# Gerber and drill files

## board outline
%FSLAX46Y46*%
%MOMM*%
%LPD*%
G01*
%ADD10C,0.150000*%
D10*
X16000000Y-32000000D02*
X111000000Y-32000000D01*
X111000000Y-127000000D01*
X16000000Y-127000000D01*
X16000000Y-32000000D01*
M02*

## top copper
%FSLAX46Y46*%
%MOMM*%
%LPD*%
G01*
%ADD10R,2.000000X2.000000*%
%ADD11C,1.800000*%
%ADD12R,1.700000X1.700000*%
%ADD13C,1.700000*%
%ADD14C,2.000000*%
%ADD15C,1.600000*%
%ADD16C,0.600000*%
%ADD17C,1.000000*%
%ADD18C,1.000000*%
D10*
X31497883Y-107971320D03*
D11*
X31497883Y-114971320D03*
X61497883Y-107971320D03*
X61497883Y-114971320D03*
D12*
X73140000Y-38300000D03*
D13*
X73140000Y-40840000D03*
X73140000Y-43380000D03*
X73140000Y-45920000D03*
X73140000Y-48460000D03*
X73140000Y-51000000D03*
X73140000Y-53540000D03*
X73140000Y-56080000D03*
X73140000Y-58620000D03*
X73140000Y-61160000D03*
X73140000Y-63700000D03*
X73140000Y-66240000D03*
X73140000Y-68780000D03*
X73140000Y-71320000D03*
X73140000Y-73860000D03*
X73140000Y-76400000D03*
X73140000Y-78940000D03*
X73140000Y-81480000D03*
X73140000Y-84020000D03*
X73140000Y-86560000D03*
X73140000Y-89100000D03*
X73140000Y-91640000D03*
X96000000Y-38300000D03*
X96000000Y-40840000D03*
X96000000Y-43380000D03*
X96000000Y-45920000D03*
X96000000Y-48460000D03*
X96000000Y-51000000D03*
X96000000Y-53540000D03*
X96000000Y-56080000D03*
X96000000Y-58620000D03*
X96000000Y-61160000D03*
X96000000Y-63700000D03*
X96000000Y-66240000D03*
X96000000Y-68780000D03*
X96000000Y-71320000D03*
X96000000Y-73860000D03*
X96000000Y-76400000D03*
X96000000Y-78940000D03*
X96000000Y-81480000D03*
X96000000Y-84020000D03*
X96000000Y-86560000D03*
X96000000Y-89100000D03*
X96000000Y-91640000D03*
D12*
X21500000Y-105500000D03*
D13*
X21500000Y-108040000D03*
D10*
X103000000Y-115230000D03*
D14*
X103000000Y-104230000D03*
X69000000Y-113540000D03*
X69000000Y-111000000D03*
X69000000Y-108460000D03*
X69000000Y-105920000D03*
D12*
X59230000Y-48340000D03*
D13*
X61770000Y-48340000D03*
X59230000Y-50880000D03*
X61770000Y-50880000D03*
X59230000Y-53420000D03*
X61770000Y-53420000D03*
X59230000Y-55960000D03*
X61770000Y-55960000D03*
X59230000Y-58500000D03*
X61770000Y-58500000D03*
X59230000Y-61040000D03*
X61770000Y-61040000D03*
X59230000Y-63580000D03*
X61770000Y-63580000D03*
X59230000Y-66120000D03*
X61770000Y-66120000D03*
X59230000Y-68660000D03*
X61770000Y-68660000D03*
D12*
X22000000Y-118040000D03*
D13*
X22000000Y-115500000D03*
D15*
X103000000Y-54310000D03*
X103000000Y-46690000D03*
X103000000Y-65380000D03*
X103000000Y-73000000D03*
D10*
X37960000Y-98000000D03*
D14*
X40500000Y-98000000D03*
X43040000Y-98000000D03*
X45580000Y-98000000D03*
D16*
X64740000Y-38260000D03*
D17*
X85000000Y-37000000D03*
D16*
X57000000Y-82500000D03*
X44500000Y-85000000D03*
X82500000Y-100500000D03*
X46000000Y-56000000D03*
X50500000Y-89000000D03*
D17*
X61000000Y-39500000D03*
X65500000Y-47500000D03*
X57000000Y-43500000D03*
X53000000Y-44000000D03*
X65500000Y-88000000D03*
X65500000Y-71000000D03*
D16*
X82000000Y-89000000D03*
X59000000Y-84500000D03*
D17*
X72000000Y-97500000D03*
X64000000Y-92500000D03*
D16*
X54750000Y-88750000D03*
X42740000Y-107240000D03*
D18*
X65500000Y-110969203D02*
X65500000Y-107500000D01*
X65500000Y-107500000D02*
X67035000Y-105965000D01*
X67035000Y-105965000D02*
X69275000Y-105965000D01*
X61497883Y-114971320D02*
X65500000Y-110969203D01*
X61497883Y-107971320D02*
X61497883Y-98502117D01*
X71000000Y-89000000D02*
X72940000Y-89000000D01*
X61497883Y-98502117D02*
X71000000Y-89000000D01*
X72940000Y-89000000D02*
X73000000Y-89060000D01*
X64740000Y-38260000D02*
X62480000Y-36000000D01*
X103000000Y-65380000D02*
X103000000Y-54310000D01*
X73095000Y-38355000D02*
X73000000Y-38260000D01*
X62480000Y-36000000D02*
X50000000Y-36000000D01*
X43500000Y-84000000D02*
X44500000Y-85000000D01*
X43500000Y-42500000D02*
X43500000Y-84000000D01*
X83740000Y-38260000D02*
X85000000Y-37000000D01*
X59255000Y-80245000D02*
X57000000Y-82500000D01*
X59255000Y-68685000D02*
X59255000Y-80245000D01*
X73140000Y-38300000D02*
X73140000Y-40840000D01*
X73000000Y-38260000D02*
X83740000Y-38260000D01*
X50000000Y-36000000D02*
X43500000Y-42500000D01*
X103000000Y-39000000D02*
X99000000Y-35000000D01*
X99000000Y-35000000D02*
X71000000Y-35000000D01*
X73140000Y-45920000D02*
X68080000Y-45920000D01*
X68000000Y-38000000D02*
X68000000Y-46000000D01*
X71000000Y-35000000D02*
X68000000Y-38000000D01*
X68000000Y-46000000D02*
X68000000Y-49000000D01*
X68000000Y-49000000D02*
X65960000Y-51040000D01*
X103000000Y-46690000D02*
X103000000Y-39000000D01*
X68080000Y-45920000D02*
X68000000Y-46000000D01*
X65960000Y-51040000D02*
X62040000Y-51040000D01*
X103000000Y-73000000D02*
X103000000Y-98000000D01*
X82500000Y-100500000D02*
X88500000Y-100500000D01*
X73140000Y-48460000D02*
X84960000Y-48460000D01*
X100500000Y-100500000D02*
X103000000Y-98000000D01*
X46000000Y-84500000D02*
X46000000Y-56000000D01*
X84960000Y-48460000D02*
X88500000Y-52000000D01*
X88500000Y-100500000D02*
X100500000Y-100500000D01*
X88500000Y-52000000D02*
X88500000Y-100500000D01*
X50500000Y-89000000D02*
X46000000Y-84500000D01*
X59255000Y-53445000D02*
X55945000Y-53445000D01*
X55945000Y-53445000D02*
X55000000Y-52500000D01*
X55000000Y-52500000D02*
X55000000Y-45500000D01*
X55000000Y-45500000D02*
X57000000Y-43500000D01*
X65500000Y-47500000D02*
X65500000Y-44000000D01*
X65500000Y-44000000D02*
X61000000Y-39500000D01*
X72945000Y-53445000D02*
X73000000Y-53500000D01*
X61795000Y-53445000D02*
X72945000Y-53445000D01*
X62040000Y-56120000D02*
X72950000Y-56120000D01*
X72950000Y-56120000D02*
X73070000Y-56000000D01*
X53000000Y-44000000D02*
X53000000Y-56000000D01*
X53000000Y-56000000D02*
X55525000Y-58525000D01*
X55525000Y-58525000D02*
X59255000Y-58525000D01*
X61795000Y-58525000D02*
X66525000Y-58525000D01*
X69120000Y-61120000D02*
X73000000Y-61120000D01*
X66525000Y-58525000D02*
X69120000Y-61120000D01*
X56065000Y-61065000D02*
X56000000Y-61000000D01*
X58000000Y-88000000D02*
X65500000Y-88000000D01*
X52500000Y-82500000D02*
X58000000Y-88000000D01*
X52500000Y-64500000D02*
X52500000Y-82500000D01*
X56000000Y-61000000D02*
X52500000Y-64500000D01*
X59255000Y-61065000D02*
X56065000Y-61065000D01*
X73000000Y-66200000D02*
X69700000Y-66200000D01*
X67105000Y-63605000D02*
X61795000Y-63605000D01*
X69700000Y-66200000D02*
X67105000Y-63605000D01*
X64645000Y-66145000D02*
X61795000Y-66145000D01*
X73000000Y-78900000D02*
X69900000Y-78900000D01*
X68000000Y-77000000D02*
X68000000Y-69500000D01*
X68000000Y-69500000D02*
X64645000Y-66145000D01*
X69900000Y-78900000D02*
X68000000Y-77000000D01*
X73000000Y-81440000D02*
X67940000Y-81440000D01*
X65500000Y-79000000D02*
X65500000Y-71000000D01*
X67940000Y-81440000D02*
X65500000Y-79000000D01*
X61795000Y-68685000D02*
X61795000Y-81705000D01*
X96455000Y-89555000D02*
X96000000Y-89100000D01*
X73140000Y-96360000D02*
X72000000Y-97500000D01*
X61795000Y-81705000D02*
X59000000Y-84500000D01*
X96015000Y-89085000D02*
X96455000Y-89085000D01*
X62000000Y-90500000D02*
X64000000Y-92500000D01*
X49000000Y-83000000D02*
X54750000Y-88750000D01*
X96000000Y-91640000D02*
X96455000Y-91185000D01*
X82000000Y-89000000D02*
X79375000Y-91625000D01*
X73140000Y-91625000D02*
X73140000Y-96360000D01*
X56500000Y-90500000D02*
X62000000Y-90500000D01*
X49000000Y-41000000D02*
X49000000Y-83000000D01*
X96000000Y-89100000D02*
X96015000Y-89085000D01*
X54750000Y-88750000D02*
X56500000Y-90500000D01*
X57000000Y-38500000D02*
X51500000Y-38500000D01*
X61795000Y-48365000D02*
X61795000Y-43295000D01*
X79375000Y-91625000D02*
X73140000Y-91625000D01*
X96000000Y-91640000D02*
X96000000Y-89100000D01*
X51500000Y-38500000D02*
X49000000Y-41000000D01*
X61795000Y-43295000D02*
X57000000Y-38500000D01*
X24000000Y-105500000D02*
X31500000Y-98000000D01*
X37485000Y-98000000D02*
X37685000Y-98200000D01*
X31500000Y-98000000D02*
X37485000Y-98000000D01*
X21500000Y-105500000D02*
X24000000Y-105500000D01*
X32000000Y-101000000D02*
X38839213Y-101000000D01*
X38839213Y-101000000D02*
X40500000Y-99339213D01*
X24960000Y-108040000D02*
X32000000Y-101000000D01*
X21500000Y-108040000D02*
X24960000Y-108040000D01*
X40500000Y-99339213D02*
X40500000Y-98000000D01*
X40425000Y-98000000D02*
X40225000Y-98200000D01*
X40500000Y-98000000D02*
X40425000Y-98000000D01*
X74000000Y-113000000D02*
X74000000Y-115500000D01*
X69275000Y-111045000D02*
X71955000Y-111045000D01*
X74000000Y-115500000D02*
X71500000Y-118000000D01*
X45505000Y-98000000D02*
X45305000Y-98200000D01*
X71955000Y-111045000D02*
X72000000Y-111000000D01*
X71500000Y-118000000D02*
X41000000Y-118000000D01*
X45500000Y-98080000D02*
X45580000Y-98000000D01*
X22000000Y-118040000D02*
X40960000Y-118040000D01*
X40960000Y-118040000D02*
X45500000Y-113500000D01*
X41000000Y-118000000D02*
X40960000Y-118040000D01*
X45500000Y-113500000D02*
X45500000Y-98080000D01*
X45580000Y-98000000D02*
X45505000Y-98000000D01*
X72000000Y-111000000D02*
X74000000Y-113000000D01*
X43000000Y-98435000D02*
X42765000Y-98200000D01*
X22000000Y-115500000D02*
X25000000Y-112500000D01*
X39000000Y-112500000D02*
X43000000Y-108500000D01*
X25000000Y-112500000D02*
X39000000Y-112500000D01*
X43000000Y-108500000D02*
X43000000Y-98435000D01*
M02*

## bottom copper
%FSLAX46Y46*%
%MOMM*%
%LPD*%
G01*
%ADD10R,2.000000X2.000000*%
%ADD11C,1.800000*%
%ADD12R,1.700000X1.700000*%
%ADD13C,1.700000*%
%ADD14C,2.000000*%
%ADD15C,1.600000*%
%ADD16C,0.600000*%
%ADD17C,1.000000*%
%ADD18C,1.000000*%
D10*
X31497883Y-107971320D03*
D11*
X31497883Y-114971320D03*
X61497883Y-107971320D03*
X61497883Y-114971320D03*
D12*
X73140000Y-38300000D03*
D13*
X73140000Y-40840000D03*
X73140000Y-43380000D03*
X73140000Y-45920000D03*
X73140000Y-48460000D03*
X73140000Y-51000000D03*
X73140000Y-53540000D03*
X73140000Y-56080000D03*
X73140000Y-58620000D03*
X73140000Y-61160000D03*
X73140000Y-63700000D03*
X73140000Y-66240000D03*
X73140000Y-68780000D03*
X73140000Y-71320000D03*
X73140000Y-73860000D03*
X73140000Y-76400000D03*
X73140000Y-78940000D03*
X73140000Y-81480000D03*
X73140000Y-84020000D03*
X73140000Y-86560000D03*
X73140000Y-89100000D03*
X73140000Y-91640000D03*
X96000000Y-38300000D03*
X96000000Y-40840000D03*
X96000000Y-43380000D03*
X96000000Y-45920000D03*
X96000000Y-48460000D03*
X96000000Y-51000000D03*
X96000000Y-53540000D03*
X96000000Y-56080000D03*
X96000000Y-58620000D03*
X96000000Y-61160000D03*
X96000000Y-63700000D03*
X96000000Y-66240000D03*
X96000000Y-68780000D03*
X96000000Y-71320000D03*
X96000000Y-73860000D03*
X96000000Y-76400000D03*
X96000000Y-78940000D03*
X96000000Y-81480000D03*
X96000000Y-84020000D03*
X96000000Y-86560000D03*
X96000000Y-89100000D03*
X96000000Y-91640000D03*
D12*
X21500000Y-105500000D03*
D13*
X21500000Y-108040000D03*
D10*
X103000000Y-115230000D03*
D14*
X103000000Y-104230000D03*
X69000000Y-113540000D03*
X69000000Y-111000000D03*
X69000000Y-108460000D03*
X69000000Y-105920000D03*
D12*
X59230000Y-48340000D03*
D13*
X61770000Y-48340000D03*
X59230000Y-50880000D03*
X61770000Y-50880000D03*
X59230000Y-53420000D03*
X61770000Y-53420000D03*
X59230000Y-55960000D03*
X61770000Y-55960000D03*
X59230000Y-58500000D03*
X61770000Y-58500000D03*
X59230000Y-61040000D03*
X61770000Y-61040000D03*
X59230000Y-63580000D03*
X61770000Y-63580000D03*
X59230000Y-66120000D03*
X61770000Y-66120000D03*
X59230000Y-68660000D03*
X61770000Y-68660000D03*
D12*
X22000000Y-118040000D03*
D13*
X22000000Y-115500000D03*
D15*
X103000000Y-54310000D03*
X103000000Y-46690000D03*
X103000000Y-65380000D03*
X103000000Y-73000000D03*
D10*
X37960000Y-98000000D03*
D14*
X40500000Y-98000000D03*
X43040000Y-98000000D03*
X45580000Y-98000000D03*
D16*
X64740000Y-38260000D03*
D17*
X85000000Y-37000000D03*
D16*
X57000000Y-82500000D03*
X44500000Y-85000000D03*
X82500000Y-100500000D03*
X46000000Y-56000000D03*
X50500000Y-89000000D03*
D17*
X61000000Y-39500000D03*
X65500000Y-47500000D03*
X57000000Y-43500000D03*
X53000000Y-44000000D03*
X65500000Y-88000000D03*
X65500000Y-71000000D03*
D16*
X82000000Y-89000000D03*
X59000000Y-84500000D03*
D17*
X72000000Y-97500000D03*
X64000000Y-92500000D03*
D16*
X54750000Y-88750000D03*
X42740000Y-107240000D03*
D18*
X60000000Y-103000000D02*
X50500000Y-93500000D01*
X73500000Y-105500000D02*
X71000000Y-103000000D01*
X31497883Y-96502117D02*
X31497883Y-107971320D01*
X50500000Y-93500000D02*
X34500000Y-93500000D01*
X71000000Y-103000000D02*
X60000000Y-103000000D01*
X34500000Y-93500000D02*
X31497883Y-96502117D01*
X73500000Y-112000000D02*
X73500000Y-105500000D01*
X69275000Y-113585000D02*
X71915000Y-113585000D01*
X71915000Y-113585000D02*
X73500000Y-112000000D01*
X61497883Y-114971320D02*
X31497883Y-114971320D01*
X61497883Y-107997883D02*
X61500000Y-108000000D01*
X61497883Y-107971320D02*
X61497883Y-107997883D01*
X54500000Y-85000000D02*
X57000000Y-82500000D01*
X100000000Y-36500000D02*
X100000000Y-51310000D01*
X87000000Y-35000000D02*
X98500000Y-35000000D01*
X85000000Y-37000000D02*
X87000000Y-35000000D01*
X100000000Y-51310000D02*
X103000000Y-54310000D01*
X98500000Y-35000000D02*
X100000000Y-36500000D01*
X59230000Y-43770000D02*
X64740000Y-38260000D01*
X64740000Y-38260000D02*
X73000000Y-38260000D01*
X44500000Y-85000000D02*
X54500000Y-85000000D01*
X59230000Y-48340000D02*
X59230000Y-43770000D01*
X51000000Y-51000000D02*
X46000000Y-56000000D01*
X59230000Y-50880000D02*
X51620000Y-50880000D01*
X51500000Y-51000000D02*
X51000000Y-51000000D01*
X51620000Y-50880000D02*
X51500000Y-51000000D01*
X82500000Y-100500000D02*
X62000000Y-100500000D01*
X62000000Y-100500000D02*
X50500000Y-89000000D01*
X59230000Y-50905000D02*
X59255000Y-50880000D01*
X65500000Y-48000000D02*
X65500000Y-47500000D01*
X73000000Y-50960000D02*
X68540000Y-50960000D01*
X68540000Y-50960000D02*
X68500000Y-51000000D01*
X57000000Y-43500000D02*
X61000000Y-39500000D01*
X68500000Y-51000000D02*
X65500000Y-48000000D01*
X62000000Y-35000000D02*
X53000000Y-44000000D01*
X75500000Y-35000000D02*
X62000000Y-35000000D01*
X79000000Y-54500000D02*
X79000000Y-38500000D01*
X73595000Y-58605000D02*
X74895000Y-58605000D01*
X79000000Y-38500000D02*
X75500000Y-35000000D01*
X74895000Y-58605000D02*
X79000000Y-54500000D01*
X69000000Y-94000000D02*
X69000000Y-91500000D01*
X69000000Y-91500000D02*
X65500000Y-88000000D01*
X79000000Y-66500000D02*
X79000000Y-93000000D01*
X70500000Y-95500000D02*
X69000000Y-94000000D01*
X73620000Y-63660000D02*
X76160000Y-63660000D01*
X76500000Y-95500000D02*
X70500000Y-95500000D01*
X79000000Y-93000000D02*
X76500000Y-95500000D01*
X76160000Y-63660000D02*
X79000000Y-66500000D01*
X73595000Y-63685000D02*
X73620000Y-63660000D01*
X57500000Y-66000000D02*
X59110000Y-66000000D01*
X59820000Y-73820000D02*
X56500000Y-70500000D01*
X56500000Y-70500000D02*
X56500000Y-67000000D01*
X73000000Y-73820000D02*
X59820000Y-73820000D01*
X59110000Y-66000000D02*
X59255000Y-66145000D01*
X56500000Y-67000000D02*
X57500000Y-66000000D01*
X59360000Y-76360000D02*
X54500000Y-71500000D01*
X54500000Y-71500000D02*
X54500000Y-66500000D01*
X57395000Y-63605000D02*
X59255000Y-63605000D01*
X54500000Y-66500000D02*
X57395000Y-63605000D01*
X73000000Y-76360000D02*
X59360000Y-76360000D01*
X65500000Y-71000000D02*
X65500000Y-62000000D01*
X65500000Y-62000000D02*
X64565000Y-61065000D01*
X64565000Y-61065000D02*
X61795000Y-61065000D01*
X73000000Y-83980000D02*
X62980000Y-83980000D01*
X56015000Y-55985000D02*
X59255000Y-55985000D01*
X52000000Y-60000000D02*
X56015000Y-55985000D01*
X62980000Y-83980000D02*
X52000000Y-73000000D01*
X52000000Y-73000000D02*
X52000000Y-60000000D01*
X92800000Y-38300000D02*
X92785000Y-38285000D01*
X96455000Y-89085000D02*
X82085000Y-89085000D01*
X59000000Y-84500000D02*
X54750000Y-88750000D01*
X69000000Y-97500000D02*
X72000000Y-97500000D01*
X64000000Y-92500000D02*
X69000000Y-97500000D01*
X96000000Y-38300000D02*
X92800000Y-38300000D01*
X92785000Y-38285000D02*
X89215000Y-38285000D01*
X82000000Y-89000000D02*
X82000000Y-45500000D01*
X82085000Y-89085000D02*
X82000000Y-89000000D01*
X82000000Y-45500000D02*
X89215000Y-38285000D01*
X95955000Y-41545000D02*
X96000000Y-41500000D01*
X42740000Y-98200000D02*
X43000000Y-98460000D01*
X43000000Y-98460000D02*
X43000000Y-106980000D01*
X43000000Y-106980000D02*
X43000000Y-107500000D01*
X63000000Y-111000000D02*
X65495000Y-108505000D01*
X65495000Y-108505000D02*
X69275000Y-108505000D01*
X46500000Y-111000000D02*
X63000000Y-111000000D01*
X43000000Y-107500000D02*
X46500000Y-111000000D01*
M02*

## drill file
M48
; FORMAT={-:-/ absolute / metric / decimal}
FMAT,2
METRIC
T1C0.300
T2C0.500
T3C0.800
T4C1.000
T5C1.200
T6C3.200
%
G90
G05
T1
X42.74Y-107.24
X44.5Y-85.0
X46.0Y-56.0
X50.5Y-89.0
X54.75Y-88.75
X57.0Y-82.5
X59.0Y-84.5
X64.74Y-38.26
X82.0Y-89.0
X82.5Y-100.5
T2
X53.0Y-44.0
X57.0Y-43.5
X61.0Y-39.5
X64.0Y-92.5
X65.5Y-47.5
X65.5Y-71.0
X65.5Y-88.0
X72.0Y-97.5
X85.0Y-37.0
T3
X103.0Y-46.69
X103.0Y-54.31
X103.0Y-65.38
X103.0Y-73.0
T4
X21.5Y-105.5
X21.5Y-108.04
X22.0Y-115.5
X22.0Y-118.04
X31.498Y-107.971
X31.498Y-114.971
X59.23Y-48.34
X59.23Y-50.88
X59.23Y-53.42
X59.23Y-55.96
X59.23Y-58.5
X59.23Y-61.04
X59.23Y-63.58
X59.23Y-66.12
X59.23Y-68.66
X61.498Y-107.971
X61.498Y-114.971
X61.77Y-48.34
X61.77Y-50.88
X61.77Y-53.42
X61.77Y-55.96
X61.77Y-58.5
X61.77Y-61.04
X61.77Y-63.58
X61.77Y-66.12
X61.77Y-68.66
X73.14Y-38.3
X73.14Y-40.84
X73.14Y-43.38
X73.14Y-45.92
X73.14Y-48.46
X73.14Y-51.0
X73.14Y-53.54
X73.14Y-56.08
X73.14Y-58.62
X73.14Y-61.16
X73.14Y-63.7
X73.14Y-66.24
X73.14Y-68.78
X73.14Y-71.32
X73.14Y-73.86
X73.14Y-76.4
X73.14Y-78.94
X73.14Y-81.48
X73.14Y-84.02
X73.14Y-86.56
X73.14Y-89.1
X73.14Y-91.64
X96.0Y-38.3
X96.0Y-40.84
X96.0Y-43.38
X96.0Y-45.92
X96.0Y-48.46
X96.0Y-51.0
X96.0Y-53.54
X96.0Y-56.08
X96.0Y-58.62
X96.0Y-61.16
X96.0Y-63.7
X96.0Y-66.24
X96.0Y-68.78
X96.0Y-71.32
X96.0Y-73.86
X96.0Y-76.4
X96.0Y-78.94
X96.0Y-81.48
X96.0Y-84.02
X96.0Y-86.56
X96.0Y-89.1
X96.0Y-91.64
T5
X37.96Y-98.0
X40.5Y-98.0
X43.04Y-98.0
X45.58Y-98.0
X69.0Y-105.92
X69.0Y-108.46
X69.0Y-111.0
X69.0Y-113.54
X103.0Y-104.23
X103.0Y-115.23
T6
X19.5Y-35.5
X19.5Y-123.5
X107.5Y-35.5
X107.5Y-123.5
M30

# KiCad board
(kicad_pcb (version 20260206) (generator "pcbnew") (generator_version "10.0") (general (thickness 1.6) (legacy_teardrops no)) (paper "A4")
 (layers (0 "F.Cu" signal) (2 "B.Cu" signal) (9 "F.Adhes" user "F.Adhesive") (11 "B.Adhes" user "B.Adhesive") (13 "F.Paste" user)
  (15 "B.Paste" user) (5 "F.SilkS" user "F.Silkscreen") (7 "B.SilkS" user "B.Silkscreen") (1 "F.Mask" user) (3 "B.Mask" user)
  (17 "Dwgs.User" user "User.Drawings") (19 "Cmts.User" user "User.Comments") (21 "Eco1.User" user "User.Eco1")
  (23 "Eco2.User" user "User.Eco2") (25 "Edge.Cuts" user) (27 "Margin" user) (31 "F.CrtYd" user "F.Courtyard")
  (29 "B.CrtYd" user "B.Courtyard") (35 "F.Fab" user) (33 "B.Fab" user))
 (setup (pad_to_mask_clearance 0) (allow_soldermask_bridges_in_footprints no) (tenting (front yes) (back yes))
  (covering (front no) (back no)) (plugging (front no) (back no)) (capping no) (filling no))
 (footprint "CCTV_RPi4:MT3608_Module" (layer "F.Cu") (at 46.497883 111.47132)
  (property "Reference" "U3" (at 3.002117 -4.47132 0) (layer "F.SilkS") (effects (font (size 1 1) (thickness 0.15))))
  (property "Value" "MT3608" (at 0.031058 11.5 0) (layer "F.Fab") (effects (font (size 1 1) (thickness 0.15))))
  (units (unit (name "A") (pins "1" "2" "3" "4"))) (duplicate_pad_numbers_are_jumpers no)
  (pad "1" thru_hole rect (at -15 -3.5) (size 2 2) (drill 1) (layers "*.Cu" "*.Mask") (remove_unused_layers no) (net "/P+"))
  (pad "2" thru_hole circle (at -15 3.5) (size 1.8 1.8) (drill 1) (layers "*.Cu" "*.Mask") (remove_unused_layers no) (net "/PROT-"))
  (pad "3" thru_hole circle (at 15 -3.5) (size 1.8 1.8) (drill 1) (layers "*.Cu" "*.Mask") (remove_unused_layers no) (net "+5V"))
  (pad "4" thru_hole circle (at 15 3.5) (size 1.8 1.8) (drill 1) (layers "*.Cu" "*.Mask") (remove_unused_layers no) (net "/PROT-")))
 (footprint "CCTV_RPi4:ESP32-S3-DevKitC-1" (layer "F.Cu") (at 84.57 66.24)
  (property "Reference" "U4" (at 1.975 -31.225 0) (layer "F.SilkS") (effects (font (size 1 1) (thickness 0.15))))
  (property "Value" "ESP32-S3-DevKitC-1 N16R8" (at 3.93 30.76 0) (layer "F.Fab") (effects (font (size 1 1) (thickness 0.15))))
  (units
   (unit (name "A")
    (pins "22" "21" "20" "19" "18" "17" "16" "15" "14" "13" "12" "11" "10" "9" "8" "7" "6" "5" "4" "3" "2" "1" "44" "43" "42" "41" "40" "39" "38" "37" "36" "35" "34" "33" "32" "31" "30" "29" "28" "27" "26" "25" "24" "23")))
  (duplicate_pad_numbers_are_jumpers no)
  (pad "1" thru_hole rect (at -11.43 -27.94) (size 1.7 1.7) (drill 1) (layers "*.Cu" "*.Mask") (remove_unused_layers no) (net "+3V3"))
  (pad "2" thru_hole circle (at -11.43 -25.4) (size 1.7 1.7) (drill 1) (layers "*.Cu" "*.Mask") (remove_unused_layers no) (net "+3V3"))
  (pad "3" thru_hole circle (at -11.43 -22.86) (size 1.7 1.7) (drill 1) (layers "*.Cu" "*.Mask") (remove_unused_layers no)
   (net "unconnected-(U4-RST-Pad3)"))
  (pad "4" thru_hole circle (at -11.43 -20.32) (size 1.7 1.7) (drill 1) (layers "*.Cu" "*.Mask") (remove_unused_layers no) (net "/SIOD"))
  (pad "5" thru_hole circle (at -11.43 -17.78) (size 1.7 1.7) (drill 1) (layers "*.Cu" "*.Mask") (remove_unused_layers no) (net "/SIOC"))
  (pad "6" thru_hole circle (at -11.43 -15.24) (size 1.7 1.7) (drill 1) (layers "*.Cu" "*.Mask") (remove_unused_layers no) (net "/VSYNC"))
  (pad "7" thru_hole circle (at -11.43 -12.7) (size 1.7 1.7) (drill 1) (layers "*.Cu" "*.Mask") (remove_unused_layers no) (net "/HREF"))
  (pad "8" thru_hole circle (at -11.43 -10.16) (size 1.7 1.7) (drill 1) (layers "*.Cu" "*.Mask") (remove_unused_layers no) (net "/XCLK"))
  (pad "9" thru_hole circle (at -11.43 -7.62) (size 1.7 1.7) (drill 1) (layers "*.Cu" "*.Mask") (remove_unused_layers no) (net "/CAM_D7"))
  (pad "10" thru_hole circle (at -11.43 -5.08) (size 1.7 1.7) (drill 1) (layers "*.Cu" "*.Mask") (remove_unused_layers no) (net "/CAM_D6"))
  (pad "11" thru_hole circle (at -11.43 -2.54) (size 1.7 1.7) (drill 1) (layers "*.Cu" "*.Mask") (remove_unused_layers no) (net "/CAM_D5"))
  (pad "12" thru_hole circle (at -11.43 0) (size 1.7 1.7) (drill 1) (layers "*.Cu" "*.Mask") (remove_unused_layers no) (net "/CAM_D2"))
  (pad "13" thru_hole circle (at -11.43 2.54) (size 1.7 1.7) (drill 1) (layers "*.Cu" "*.Mask") (remove_unused_layers no)
   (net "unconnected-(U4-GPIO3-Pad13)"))
  (pad "14" thru_hole circle (at -11.43 5.08) (size 1.7 1.7) (drill 1) (layers "*.Cu" "*.Mask") (remove_unused_layers no)
   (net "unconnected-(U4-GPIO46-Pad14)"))
  (pad "15" thru_hole circle (at -11.43 7.62) (size 1.7 1.7) (drill 1) (layers "*.Cu" "*.Mask") (remove_unused_layers no) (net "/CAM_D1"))
  (pad "16" thru_hole circle (at -11.43 10.16) (size 1.7 1.7) (drill 1) (layers "*.Cu" "*.Mask") (remove_unused_layers no) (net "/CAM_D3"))
  (pad "17" thru_hole circle (at -11.43 12.7) (size 1.7 1.7) (drill 1) (layers "*.Cu" "*.Mask") (remove_unused_layers no) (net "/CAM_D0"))
  (pad "18" thru_hole circle (at -11.43 15.24) (size 1.7 1.7) (drill 1) (layers "*.Cu" "*.Mask") (remove_unused_layers no) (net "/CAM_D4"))
  (pad "19" thru_hole circle (at -11.43 17.78) (size 1.7 1.7) (drill 1) (layers "*.Cu" "*.Mask") (remove_unused_layers no) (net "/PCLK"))
  (pad "20" thru_hole circle (at -11.43 20.32) (size 1.7 1.7) (drill 1) (layers "*.Cu" "*.Mask") (remove_unused_layers no)
   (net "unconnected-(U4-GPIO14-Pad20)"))
  (pad "21" thru_hole circle (at -11.43 22.86) (size 1.7 1.7) (drill 1) (layers "*.Cu" "*.Mask") (remove_unused_layers no) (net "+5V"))
  (pad "22" thru_hole circle (at -11.43 25.4) (size 1.7 1.7) (drill 1) (layers "*.Cu" "*.Mask") (remove_unused_layers no) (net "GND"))
  (pad "23" thru_hole circle (at 11.43 -27.94) (size 1.7 1.7) (drill 1) (layers "*.Cu" "*.Mask") (remove_unused_layers no) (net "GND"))
  (pad "24" thru_hole circle (at 11.43 -25.4) (size 1.7 1.7) (drill 1) (layers "*.Cu" "*.Mask") (remove_unused_layers no)
   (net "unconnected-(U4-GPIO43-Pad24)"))
  (pad "25" thru_hole circle (at 11.43 -22.86) (size 1.7 1.7) (drill 1) (layers "*.Cu" "*.Mask") (remove_unused_layers no)
   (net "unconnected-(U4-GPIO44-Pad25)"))
  (pad "26" thru_hole circle (at 11.43 -20.32) (size 1.7 1.7) (drill 1) (layers "*.Cu" "*.Mask") (remove_unused_layers no)
   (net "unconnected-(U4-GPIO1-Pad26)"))
  (pad "27" thru_hole circle (at 11.43 -17.78) (size 1.7 1.7) (drill 1) (layers "*.Cu" "*.Mask") (remove_unused_layers no)
   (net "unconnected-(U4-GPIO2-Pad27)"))
  (pad "28" thru_hole circle (at 11.43 -15.24) (size 1.7 1.7) (drill 1) (layers "*.Cu" "*.Mask") (remove_unused_layers no)
   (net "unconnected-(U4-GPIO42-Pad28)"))
  (pad "29" thru_hole circle (at 11.43 -12.7) (size 1.7 1.7) (drill 1) (layers "*.Cu" "*.Mask") (remove_unused_layers no)
   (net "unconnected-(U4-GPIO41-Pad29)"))
  (pad "30" thru_hole circle (at 11.43 -10.16) (size 1.7 1.7) (drill 1) (layers "*.Cu" "*.Mask") (remove_unused_layers no)
   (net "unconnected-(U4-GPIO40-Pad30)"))
  (pad "31" thru_hole circle (at 11.43 -7.62) (size 1.7 1.7) (drill 1) (layers "*.Cu" "*.Mask") (remove_unused_layers no)
   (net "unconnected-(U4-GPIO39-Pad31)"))
  (pad "32" thru_hole circle (at 11.43 -5.08) (size 1.7 1.7) (drill 1) (layers "*.Cu" "*.Mask") (remove_unused_layers no)
   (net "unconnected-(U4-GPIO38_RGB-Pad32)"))
  (pad "33" thru_hole circle (at 11.43 -2.54) (size 1.7 1.7) (drill 1) (layers "*.Cu" "*.Mask") (remove_unused_layers no)
   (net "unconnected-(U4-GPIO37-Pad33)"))
  (pad "34" thru_hole circle (at 11.43 0) (size 1.7 1.7) (drill 1) (layers "*.Cu" "*.Mask") (remove_unused_layers no)
   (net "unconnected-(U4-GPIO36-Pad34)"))
  (pad "35" thru_hole circle (at 11.43 2.54) (size 1.7 1.7) (drill 1) (layers "*.Cu" "*.Mask") (remove_unused_layers no)
   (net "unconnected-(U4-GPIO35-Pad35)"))
  (pad "36" thru_hole circle (at 11.43 5.08) (size 1.7 1.7) (drill 1) (layers "*.Cu" "*.Mask") (remove_unused_layers no)
   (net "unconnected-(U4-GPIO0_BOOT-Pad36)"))
  (pad "37" thru_hole circle (at 11.43 7.62) (size 1.7 1.7) (drill 1) (layers "*.Cu" "*.Mask") (remove_unused_layers no)
   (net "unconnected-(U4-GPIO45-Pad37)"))
  (pad "38" thru_hole circle (at 11.43 10.16) (size 1.7 1.7) (drill 1) (layers "*.Cu" "*.Mask") (remove_unused_layers no)
   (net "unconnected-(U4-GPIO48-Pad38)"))
  (pad "39" thru_hole circle (at 11.43 12.7) (size 1.7 1.7) (drill 1) (layers "*.Cu" "*.Mask") (remove_unused_layers no)
   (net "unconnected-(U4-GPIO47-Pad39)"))
  (pad "40" thru_hole circle (at 11.43 15.24) (size 1.7 1.7) (drill 1) (layers "*.Cu" "*.Mask") (remove_unused_layers no)
   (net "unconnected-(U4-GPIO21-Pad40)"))
  (pad "41" thru_hole circle (at 11.43 17.78) (size 1.7 1.7) (drill 1) (layers "*.Cu" "*.Mask") (remove_unused_layers no)
   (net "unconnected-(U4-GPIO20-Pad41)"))
  (pad "42" thru_hole circle (at 11.43 20.32) (size 1.7 1.7) (drill 1) (layers "*.Cu" "*.Mask") (remove_unused_layers no)
   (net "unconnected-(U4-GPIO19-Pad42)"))
  (pad "43" thru_hole circle (at 11.43 22.86) (size 1.7 1.7) (drill 1) (layers "*.Cu" "*.Mask") (remove_unused_layers no) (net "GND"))
  (pad "44" thru_hole circle (at 11.43 25.4) (size 1.7 1.7) (drill 1) (layers "*.Cu" "*.Mask") (remove_unused_layers no) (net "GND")))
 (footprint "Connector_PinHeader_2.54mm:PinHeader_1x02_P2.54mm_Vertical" (layer "F.Cu") (at 21.5 105.5)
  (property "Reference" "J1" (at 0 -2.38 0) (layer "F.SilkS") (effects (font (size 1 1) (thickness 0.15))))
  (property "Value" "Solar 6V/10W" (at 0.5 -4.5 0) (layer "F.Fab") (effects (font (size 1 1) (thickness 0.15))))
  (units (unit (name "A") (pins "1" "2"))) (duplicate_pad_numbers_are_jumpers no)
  (pad "1" thru_hole rect (at 0 0) (size 1.7 1.7) (drill 1) (layers "*.Cu" "*.Mask") (remove_unused_layers no) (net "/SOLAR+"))
  (pad "2" thru_hole circle (at 0 2.54) (size 1.7 1.7) (drill 1) (layers "*.Cu" "*.Mask") (remove_unused_layers no) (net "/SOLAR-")))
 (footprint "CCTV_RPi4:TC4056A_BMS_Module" (layer "F.Cu") (at 86 109.73 180)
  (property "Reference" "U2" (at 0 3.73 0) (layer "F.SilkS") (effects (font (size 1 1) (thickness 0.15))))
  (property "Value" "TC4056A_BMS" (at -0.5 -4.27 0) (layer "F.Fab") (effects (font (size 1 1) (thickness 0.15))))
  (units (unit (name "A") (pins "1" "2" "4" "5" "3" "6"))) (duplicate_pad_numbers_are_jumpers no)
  (pad "1" thru_hole rect (at -17 -5.5 180) (size 2 2) (drill 1.2) (layers "*.Cu" "*.Mask") (remove_unused_layers no)
   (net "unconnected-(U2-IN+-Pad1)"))
  (pad "2" thru_hole circle (at -17 5.5 180) (size 2 2) (drill 1.2) (layers "*.Cu" "*.Mask") (remove_unused_layers no)
   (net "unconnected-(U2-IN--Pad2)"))
  (pad "3" thru_hole circle (at 17 -3.81 180) (size 2 2) (drill 1.2) (layers "*.Cu" "*.Mask") (remove_unused_layers no) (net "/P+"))
  (pad "4" thru_hole circle (at 17 -1.27 180) (size 2 2) (drill 1.2) (layers "*.Cu" "*.Mask") (remove_unused_layers no) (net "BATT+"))
  (pad "5" thru_hole circle (at 17 1.27 180) (size 2 2) (drill 1.2) (layers "*.Cu" "*.Mask") (remove_unused_layers no) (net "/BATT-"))
  (pad "6" thru_hole circle (at 17 3.81 180) (size 2 2) (drill 1.2) (layers "*.Cu" "*.Mask") (remove_unused_layers no) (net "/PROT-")))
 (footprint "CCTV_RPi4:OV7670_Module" (layer "F.Cu") (at 60.5 58.5)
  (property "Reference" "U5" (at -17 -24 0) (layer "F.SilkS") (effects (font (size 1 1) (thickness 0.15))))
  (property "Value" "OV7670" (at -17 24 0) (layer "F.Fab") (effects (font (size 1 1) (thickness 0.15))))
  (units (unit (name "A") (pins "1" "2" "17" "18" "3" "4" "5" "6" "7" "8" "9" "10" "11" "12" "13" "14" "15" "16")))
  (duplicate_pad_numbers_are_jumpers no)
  (pad "1" thru_hole rect (at -1.27 -10.16) (size 1.7 1.7) (drill 1) (layers "*.Cu" "*.Mask") (remove_unused_layers no) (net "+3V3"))
  (pad "2" thru_hole circle (at 1.27 -10.16) (size 1.7 1.7) (drill 1) (layers "*.Cu" "*.Mask") (remove_unused_layers no) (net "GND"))
  (pad "3" thru_hole circle (at -1.27 -7.62) (size 1.7 1.7) (drill 1) (layers "*.Cu" "*.Mask") (remove_unused_layers no) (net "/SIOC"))
  (pad "4" thru_hole circle (at 1.27 -7.62) (size 1.7 1.7) (drill 1) (layers "*.Cu" "*.Mask") (remove_unused_layers no) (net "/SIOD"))
  (pad "5" thru_hole circle (at -1.27 -5.08) (size 1.7 1.7) (drill 1) (layers "*.Cu" "*.Mask") (remove_unused_layers no) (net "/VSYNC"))
  (pad "6" thru_hole circle (at 1.27 -5.08) (size 1.7 1.7) (drill 1) (layers "*.Cu" "*.Mask") (remove_unused_layers no) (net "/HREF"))
  (pad "7" thru_hole circle (at -1.27 -2.54) (size 1.7 1.7) (drill 1) (layers "*.Cu" "*.Mask") (remove_unused_layers no) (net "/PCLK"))
  (pad "8" thru_hole circle (at 1.27 -2.54) (size 1.7 1.7) (drill 1) (layers "*.Cu" "*.Mask") (remove_unused_layers no) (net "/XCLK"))
  (pad "9" thru_hole circle (at -1.27 0) (size 1.7 1.7) (drill 1) (layers "*.Cu" "*.Mask") (remove_unused_layers no) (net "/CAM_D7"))
  (pad "10" thru_hole circle (at 1.27 0) (size 1.7 1.7) (drill 1) (layers "*.Cu" "*.Mask") (remove_unused_layers no) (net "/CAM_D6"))
  (pad "11" thru_hole circle (at -1.27 2.54) (size 1.7 1.7) (drill 1) (layers "*.Cu" "*.Mask") (remove_unused_layers no) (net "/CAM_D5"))
  (pad "12" thru_hole circle (at 1.27 2.54) (size 1.7 1.7) (drill 1) (layers "*.Cu" "*.Mask") (remove_unused_layers no) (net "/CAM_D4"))
  (pad "13" thru_hole circle (at -1.27 5.08) (size 1.7 1.7) (drill 1) (layers "*.Cu" "*.Mask") (remove_unused_layers no) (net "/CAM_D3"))
  (pad "14" thru_hole circle (at 1.27 5.08) (size 1.7 1.7) (drill 1) (layers "*.Cu" "*.Mask") (remove_unused_layers no) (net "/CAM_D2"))
  (pad "15" thru_hole circle (at -1.27 7.62) (size 1.7 1.7) (drill 1) (layers "*.Cu" "*.Mask") (remove_unused_layers no) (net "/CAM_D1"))
  (pad "16" thru_hole circle (at 1.27 7.62) (size 1.7 1.7) (drill 1) (layers "*.Cu" "*.Mask") (remove_unused_layers no) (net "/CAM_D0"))
  (pad "17" thru_hole circle (at -1.27 10.16) (size 1.7 1.7) (drill 1) (layers "*.Cu" "*.Mask") (remove_unused_layers no) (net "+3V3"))
  (pad "18" thru_hole circle (at 1.27 10.16) (size 1.7 1.7) (drill 1) (layers "*.Cu" "*.Mask") (remove_unused_layers no) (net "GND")))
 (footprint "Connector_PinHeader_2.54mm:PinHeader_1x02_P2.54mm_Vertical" (layer "F.Cu") (at 22 118.04 180)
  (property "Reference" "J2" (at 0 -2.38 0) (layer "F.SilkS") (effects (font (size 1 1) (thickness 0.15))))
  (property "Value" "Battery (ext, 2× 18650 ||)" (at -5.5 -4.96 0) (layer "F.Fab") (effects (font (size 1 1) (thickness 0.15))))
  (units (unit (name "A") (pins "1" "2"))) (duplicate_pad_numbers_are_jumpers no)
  (pad "1" thru_hole rect (at 0 0 180) (size 1.7 1.7) (drill 1) (layers "*.Cu" "*.Mask") (remove_unused_layers no) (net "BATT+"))
  (pad "2" thru_hole circle (at 0 2.54 180) (size 1.7 1.7) (drill 1) (layers "*.Cu" "*.Mask") (remove_unused_layers no) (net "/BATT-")))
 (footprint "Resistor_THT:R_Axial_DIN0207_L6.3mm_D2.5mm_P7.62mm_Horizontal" (layer "F.Cu") (at 103 54.31 90)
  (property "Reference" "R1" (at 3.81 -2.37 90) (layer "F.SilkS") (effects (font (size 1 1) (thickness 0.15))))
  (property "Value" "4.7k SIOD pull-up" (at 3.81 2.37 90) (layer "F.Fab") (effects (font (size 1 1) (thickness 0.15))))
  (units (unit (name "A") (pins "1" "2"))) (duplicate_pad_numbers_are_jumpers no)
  (pad "1" thru_hole circle (at 0 0 90) (size 1.6 1.6) (drill 0.8) (layers "*.Cu" "*.Mask") (remove_unused_layers no) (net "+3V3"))
  (pad "2" thru_hole circle (at 7.62 0 90) (size 1.6 1.6) (drill 0.8) (layers "*.Cu" "*.Mask") (remove_unused_layers no) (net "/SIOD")))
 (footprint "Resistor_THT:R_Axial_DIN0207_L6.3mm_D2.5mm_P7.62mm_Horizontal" (layer "F.Cu") (at 103 65.38 -90)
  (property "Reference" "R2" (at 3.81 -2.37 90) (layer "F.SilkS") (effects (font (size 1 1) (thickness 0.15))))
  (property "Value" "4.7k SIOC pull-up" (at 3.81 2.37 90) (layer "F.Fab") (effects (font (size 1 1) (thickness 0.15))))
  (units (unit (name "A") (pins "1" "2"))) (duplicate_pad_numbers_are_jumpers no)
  (pad "1" thru_hole circle (at 0 0 270) (size 1.6 1.6) (drill 0.8) (layers "*.Cu" "*.Mask") (remove_unused_layers no) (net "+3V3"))
  (pad "2" thru_hole circle (at 7.62 0 270) (size 1.6 1.6) (drill 0.8) (layers "*.Cu" "*.Mask") (remove_unused_layers no) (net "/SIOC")))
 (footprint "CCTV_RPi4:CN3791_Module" (layer "F.Cu") (at 40.5 90.5)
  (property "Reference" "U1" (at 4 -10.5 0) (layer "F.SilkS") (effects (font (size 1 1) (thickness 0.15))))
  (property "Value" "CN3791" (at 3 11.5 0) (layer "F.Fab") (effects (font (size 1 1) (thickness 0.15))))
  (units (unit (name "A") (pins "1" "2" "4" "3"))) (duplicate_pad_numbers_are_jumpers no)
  (pad "1" thru_hole rect (at -2.54 7.5) (size 2 2) (drill 1.2) (layers "*.Cu" "*.Mask") (remove_unused_layers no) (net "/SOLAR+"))
  (pad "2" thru_hole circle (at 0 7.5) (size 2 2) (drill 1.2) (layers "*.Cu" "*.Mask") (remove_unused_layers no) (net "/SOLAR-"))
  (pad "3" thru_hole circle (at 2.54 7.5) (size 2 2) (drill 1.2) (layers "*.Cu" "*.Mask") (remove_unused_layers no) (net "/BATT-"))
  (pad "4" thru_hole circle (at 5.08 7.5) (size 2 2) (drill 1.2) (layers "*.Cu" "*.Mask") (remove_unused_layers no) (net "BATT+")))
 (gr_rect (start 16 32) (end 111 127) (stroke (width 0.15) (type solid)) (fill no) (layer "Edge.Cuts"))
 (segment (start 60 103) (end 50.5 93.5) (width 1) (layer "B.Cu") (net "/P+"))
 (segment (start 73.5 105.5) (end 71 103) (width 1) (layer "B.Cu") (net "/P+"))
 (segment (start 31.497883 96.502117) (end 31.497883 107.97132) (width 1) (layer "B.Cu") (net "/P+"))
 (segment (start 50.5 93.5) (end 34.5 93.5) (width 1) (layer "B.Cu") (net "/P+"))
 (segment (start 71 103) (end 60 103) (width 1) (layer "B.Cu") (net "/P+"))
 (segment (start 34.5 93.5) (end 31.497883 96.502117) (width 1) (layer "B.Cu") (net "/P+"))
 (segment (start 73.5 112) (end 73.5 105.5) (width 1) (layer "B.Cu") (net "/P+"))
 (segment (start 69.275 113.585) (end 71.915 113.585) (width 1) (layer "B.Cu") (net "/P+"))
 (segment (start 71.915 113.585) (end 73.5 112) (width 1) (layer "B.Cu") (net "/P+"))
 (segment (start 65.5 110.969203) (end 65.5 107.5) (width 1) (layer "F.Cu") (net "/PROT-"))
 (segment (start 65.5 107.5) (end 67.035 105.965) (width 1) (layer "F.Cu") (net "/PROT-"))
 (segment (start 67.035 105.965) (end 69.275 105.965) (width 1) (layer "F.Cu") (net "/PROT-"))
 (segment (start 61.497883 114.97132) (end 65.5 110.969203) (width 1) (layer "F.Cu") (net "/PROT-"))
 (segment (start 61.497883 114.97132) (end 31.497883 114.97132) (width 1) (layer "B.Cu") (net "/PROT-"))
 (segment (start 61.497883 107.97132) (end 61.497883 98.502117) (width 1) (layer "F.Cu") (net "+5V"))
 (segment (start 71 89) (end 72.94 89) (width 1) (layer "F.Cu") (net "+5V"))
 (segment (start 61.497883 98.502117) (end 71 89) (width 1) (layer "F.Cu") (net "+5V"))
 (segment (start 72.94 89) (end 73 89.06) (width 1) (layer "F.Cu") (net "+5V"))
 (segment (start 61.497883 107.997883) (end 61.5 108) (width 1) (layer "B.Cu") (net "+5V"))
 (segment (start 61.497883 107.97132) (end 61.497883 107.997883) (width 1) (layer "B.Cu") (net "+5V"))
 (segment (start 64.74 38.26) (end 62.48 36) (width 1) (layer "F.Cu") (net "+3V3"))
 (segment (start 103 65.38) (end 103 54.31) (width 1) (layer "F.Cu") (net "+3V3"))
 (segment (start 73.095 38.355) (end 73 38.26) (width 1) (layer "F.Cu") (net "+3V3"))
 (segment (start 62.48 36) (end 50 36) (width 1) (layer "F.Cu") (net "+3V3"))
 (segment (start 43.5 84) (end 44.5 85) (width 1) (layer "F.Cu") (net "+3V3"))
 (segment (start 43.5 42.5) (end 43.5 84) (width 1) (layer "F.Cu") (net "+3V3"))
 (segment (start 83.74 38.26) (end 85 37) (width 1) (layer "F.Cu") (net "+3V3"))
 (segment (start 59.255 80.245) (end 57 82.5) (width 1) (layer "F.Cu") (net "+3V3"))
 (segment (start 59.255 68.685) (end 59.255 80.245) (width 1) (layer "F.Cu") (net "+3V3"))
 (segment (start 73.14 38.3) (end 73.14 40.84) (width 1) (layer "F.Cu") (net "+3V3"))
 (segment (start 73 38.26) (end 83.74 38.26) (width 1) (layer "F.Cu") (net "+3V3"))
 (segment (start 50 36) (end 43.5 42.5) (width 1) (layer "F.Cu") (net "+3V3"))
 (via (at 64.74 38.26) (size 0.6) (drill 0.3) (layers "F.Cu" "B.Cu") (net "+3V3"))
 (via (at 85 37) (size 1) (drill 0.5) (layers "F.Cu" "B.Cu") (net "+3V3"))
 (via (at 57 82.5) (size 0.6) (drill 0.3) (layers "F.Cu" "B.Cu") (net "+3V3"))
 (via (at 44.5 85) (size 0.6) (drill 0.3) (layers "F.Cu" "B.Cu") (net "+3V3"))
 (segment (start 54.5 85) (end 57 82.5) (width 1) (layer "B.Cu") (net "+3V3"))
 (segment (start 100 36.5) (end 100 51.31) (width 1) (layer "B.Cu") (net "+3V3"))
 (segment (start 87 35) (end 98.5 35) (width 1) (layer "B.Cu") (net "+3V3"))
 (segment (start 85 37) (end 87 35) (width 1) (layer "B.Cu") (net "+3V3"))
 (segment (start 100 51.31) (end 103 54.31) (width 1) (layer "B.Cu") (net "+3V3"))
 (segment (start 98.5 35) (end 100 36.5) (width 1) (layer "B.Cu") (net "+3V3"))
 (segment (start 59.23 43.77) (end 64.74 38.26) (width 1) (layer "B.Cu") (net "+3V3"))
 (segment (start 64.74 38.26) (end 73 38.26) (width 1) (layer "B.Cu") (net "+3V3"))
 (segment (start 44.5 85) (end 54.5 85) (width 1) (layer "B.Cu") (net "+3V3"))
 (segment (start 59.23 48.34) (end 59.23 43.77) (width 1) (layer "B.Cu") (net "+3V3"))
 (segment (start 103 39) (end 99 35) (width 1) (layer "F.Cu") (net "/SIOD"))
 (segment (start 99 35) (end 71 35) (width 1) (layer "F.Cu") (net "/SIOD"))
 (segment (start 73.14 45.92) (end 68.08 45.92) (width 1) (layer "F.Cu") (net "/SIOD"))
 (segment (start 68 38) (end 68 46) (width 1) (layer "F.Cu") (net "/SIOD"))
 (segment (start 71 35) (end 68 38) (width 1) (layer "F.Cu") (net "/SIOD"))
 (segment (start 68 46) (end 68 49) (width 1) (layer "F.Cu") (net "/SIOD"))
 (segment (start 68 49) (end 65.96 51.04) (width 1) (layer "F.Cu") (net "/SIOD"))
 (segment (start 103 46.69) (end 103 39) (width 1) (layer "F.Cu") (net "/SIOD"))
 (segment (start 68.08 45.92) (end 68 46) (width 1) (layer "F.Cu") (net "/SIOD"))
 (segment (start 65.96 51.04) (end 62.04 51.04) (width 1) (layer "F.Cu") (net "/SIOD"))
 (segment (start 103 73) (end 103 98) (width 1) (layer "F.Cu") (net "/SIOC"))
 (segment (start 82.5 100.5) (end 88.5 100.5) (width 1) (layer "F.Cu") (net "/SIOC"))
 (segment (start 73.14 48.46) (end 84.96 48.46) (width 1) (layer "F.Cu") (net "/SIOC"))
 (segment (start 100.5 100.5) (end 103 98) (width 1) (layer "F.Cu") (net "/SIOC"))
 (segment (start 46 84.5) (end 46 56) (width 1) (layer "F.Cu") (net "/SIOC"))
 (segment (start 84.96 48.46) (end 88.5 52) (width 1) (layer "F.Cu") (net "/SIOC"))
 (segment (start 88.5 100.5) (end 100.5 100.5) (width 1) (layer "F.Cu") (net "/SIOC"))
 (segment (start 88.5 52) (end 88.5 100.5) (width 1) (layer "F.Cu") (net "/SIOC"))
 (segment (start 50.5 89) (end 46 84.5) (width 1) (layer "F.Cu") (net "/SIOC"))
 (via (at 82.5 100.5) (size 0.6) (drill 0.3) (layers "F.Cu" "B.Cu") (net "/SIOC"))
 (via (at 46 56) (size 0.6) (drill 0.3) (layers "F.Cu" "B.Cu") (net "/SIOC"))
 (via (at 50.5 89) (size 0.6) (drill 0.3) (layers "F.Cu" "B.Cu") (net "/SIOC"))
 (segment (start 51 51) (end 46 56) (width 1) (layer "B.Cu") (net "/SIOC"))
 (segment (start 59.23 50.88) (end 51.62 50.88) (width 1) (layer "B.Cu") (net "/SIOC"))
 (segment (start 51.5 51) (end 51 51) (width 1) (layer "B.Cu") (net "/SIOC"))
 (segment (start 51.62 50.88) (end 51.5 51) (width 1) (layer "B.Cu") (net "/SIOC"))
 (segment (start 82.5 100.5) (end 62 100.5) (width 1) (layer "B.Cu") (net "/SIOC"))
 (segment (start 62 100.5) (end 50.5 89) (width 1) (layer "B.Cu") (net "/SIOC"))
 (segment (start 59.23 50.905) (end 59.255 50.88) (width 1) (layer "B.Cu") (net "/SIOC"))
 (segment (start 59.255 53.445) (end 55.945 53.445) (width 1) (layer "F.Cu") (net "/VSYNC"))
 (segment (start 55.945 53.445) (end 55 52.5) (width 1) (layer "F.Cu") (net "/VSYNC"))
 (segment (start 55 52.5) (end 55 45.5) (width 1) (layer "F.Cu") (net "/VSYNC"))
 (segment (start 55 45.5) (end 57 43.5) (width 1) (layer "F.Cu") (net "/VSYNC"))
 (segment (start 65.5 47.5) (end 65.5 44) (width 1) (layer "F.Cu") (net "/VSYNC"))
 (segment (start 65.5 44) (end 61 39.5) (width 1) (layer "F.Cu") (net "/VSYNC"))
 (via (at 61 39.5) (size 1) (drill 0.5) (layers "F.Cu" "B.Cu") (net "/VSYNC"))
 (via (at 65.5 47.5) (size 1) (drill 0.5) (layers "F.Cu" "B.Cu") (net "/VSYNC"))
 (via (at 57 43.5) (size 1) (drill 0.5) (layers "F.Cu" "B.Cu") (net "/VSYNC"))
 (segment (start 65.5 48) (end 65.5 47.5) (width 1) (layer "B.Cu") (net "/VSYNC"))
 (segment (start 73 50.96) (end 68.54 50.96) (width 1) (layer "B.Cu") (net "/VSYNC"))
 (segment (start 68.54 50.96) (end 68.5 51) (width 1) (layer "B.Cu") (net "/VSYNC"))
 (segment (start 57 43.5) (end 61 39.5) (width 1) (layer "B.Cu") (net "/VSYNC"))
 (segment (start 68.5 51) (end 65.5 48) (width 1) (layer "B.Cu") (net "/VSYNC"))
 (segment (start 72.945 53.445) (end 73 53.5) (width 1) (layer "F.Cu") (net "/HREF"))
 (segment (start 61.795 53.445) (end 72.945 53.445) (width 1) (layer "F.Cu") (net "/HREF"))
 (segment (start 62.04 56.12) (end 72.95 56.12) (width 1) (layer "F.Cu") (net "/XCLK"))
 (segment (start 72.95 56.12) (end 73.07 56) (width 1) (layer "F.Cu") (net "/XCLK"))
 (segment (start 53 44) (end 53 56) (width 1) (layer "F.Cu") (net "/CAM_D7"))
 (segment (start 53 56) (end 55.525 58.525) (width 1) (layer "F.Cu") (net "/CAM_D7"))
 (segment (start 55.525 58.525) (end 59.255 58.525) (width 1) (layer "F.Cu") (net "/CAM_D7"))
 (via (at 53 44) (size 1) (drill 0.5) (layers "F.Cu" "B.Cu") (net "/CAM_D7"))
 (segment (start 62 35) (end 53 44) (width 1) (layer "B.Cu") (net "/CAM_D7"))
 (segment (start 75.5 35) (end 62 35) (width 1) (layer "B.Cu") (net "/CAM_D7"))
 (segment (start 79 54.5) (end 79 38.5) (width 1) (layer "B.Cu") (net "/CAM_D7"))
 (segment (start 73.595 58.605) (end 74.895 58.605) (width 1) (layer "B.Cu") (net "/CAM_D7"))
 (segment (start 79 38.5) (end 75.5 35) (width 1) (layer "B.Cu") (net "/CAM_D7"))
 (segment (start 74.895 58.605) (end 79 54.5) (width 1) (layer "B.Cu") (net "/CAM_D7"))
 (segment (start 61.795 58.525) (end 66.525 58.525) (width 1) (layer "F.Cu") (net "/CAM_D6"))
 (segment (start 69.12 61.12) (end 73 61.12) (width 1) (layer "F.Cu") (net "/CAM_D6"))
 (segment (start 66.525 58.525) (end 69.12 61.12) (width 1) (layer "F.Cu") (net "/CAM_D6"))
 (segment (start 56.065 61.065) (end 56 61) (width 1) (layer "F.Cu") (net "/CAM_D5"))
 (segment (start 58 88) (end 65.5 88) (width 1) (layer "F.Cu") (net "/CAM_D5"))
 (segment (start 52.5 82.5) (end 58 88) (width 1) (layer "F.Cu") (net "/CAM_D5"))
 (segment (start 52.5 64.5) (end 52.5 82.5) (width 1) (layer "F.Cu") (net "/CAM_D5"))
 (segment (start 56 61) (end 52.5 64.5) (width 1) (layer "F.Cu") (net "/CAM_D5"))
 (segment (start 59.255 61.065) (end 56.065 61.065) (width 1) (layer "F.Cu") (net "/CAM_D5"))
 (via (at 65.5 88) (size 1) (drill 0.5) (layers "F.Cu" "B.Cu") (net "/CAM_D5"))
 (segment (start 69 94) (end 69 91.5) (width 1) (layer "B.Cu") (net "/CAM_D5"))
 (segment (start 69 91.5) (end 65.5 88) (width 1) (layer "B.Cu") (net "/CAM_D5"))
 (segment (start 79 66.5) (end 79 93) (width 1) (layer "B.Cu") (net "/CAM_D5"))
 (segment (start 70.5 95.5) (end 69 94) (width 1) (layer "B.Cu") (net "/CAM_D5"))
 (segment (start 73.62 63.66) (end 76.16 63.66) (width 1) (layer "B.Cu") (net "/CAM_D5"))
 (segment (start 76.5 95.5) (end 70.5 95.5) (width 1) (layer "B.Cu") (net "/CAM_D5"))
 (segment (start 79 93) (end 76.5 95.5) (width 1) (layer "B.Cu") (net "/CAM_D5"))
 (segment (start 76.16 63.66) (end 79 66.5) (width 1) (layer "B.Cu") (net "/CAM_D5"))
 (segment (start 73.595 63.685) (end 73.62 63.66) (width 1) (layer "B.Cu") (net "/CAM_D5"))
 (segment (start 73 66.2) (end 69.7 66.2) (width 1) (layer "F.Cu") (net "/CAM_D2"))
 (segment (start 67.105 63.605) (end 61.795 63.605) (width 1) (layer "F.Cu") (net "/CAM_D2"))
 (segment (start 69.7 66.2) (end 67.105 63.605) (width 1) (layer "F.Cu") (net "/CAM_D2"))
 (segment (start 57.5 66) (end 59.11 66) (width 1) (layer "B.Cu") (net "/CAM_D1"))
 (segment (start 59.82 73.82) (end 56.5 70.5) (width 1) (layer "B.Cu") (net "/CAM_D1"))
 (segment (start 56.5 70.5) (end 56.5 67) (width 1) (layer "B.Cu") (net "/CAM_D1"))
 (segment (start 73 73.82) (end 59.82 73.82) (width 1) (layer "B.Cu") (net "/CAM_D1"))
 (segment (start 59.11 66) (end 59.255 66.145) (width 1) (layer "B.Cu") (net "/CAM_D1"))
 (segment (start 56.5 67) (end 57.5 66) (width 1) (layer "B.Cu") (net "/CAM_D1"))
 (segment (start 59.36 76.36) (end 54.5 71.5) (width 1) (layer "B.Cu") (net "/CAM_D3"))
 (segment (start 54.5 71.5) (end 54.5 66.5) (width 1) (layer "B.Cu") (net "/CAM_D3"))
 (segment (start 57.395 63.605) (end 59.255 63.605) (width 1) (layer "B.Cu") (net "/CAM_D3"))
 (segment (start 54.5 66.5) (end 57.395 63.605) (width 1) (layer "B.Cu") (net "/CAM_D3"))
 (segment (start 73 76.36) (end 59.36 76.36) (width 1) (layer "B.Cu") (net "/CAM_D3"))
 (segment (start 64.645 66.145) (end 61.795 66.145) (width 1) (layer "F.Cu") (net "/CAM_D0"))
 (segment (start 73 78.9) (end 69.9 78.9) (width 1) (layer "F.Cu") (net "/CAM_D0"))
 (segment (start 68 77) (end 68 69.5) (width 1) (layer "F.Cu") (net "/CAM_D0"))
 (segment (start 68 69.5) (end 64.645 66.145) (width 1) (layer "F.Cu") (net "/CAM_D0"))
 (segment (start 69.9 78.9) (end 68 77) (width 1) (layer "F.Cu") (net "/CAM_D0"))
 (segment (start 73 81.44) (end 67.94 81.44) (width 1) (layer "F.Cu") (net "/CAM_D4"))
 (segment (start 65.5 79) (end 65.5 71) (width 1) (layer "F.Cu") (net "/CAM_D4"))
 (segment (start 67.94 81.44) (end 65.5 79) (width 1) (layer "F.Cu") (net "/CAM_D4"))
 (via (at 65.5 71) (size 1) (drill 0.5) (layers "F.Cu" "B.Cu") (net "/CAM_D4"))
 (segment (start 65.5 71) (end 65.5 62) (width 1) (layer "B.Cu") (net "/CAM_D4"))
 (segment (start 65.5 62) (end 64.565 61.065) (width 1) (layer "B.Cu") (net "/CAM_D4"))
 (segment (start 64.565 61.065) (end 61.795 61.065) (width 1) (layer "B.Cu") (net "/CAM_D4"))
 (segment (start 73 83.98) (end 62.98 83.98) (width 1) (layer "B.Cu") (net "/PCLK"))
 (segment (start 56.015 55.985) (end 59.255 55.985) (width 1) (layer "B.Cu") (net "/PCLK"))
 (segment (start 52 60) (end 56.015 55.985) (width 1) (layer "B.Cu") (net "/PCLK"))
 (segment (start 62.98 83.98) (end 52 73) (width 1) (layer "B.Cu") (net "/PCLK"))
 (segment (start 52 73) (end 52 60) (width 1) (layer "B.Cu") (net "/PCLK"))
 (segment (start 61.795 68.685) (end 61.795 81.705) (width 1) (layer "F.Cu") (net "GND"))
 (segment (start 96.455 89.555) (end 96 89.1) (width 1) (layer "F.Cu") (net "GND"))
 (segment (start 73.14 96.36) (end 72 97.5) (width 1) (layer "F.Cu") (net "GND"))
 (segment (start 61.795 81.705) (end 59 84.5) (width 1) (layer "F.Cu") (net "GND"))
 (segment (start 96.015 89.085) (end 96.455 89.085) (width 1) (layer "F.Cu") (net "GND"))
 (segment (start 62 90.5) (end 64 92.5) (width 1) (layer "F.Cu") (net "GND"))
 (segment (start 49 83) (end 54.75 88.75) (width 1) (layer "F.Cu") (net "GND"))
 (segment (start 96 91.64) (end 96.455 91.185) (width 1) (layer "F.Cu") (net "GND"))
 (segment (start 82 89) (end 79.375 91.625) (width 1) (layer "F.Cu") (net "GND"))
 (segment (start 73.14 91.625) (end 73.14 96.36) (width 1) (layer "F.Cu") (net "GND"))
 (segment (start 56.5 90.5) (end 62 90.5) (width 1) (layer "F.Cu") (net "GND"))
 (segment (start 49 41) (end 49 83) (width 1) (layer "F.Cu") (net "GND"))
 (segment (start 96 89.1) (end 96.015 89.085) (width 1) (layer "F.Cu") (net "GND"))
 (segment (start 54.75 88.75) (end 56.5 90.5) (width 1) (layer "F.Cu") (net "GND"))
 (segment (start 57 38.5) (end 51.5 38.5) (width 1) (layer "F.Cu") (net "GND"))
 (segment (start 61.795 48.365) (end 61.795 43.295) (width 1) (layer "F.Cu") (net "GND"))
 (segment (start 79.375 91.625) (end 73.14 91.625) (width 1) (layer "F.Cu") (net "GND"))
 (segment (start 96 91.64) (end 96 89.1) (width 1) (layer "F.Cu") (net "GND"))
 (segment (start 51.5 38.5) (end 49 41) (width 1) (layer "F.Cu") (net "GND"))
 (segment (start 61.795 43.295) (end 57 38.5) (width 1) (layer "F.Cu") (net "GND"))
 (via (at 82 89) (size 0.6) (drill 0.3) (layers "F.Cu" "B.Cu") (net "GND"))
 (via (at 59 84.5) (size 0.6) (drill 0.3) (layers "F.Cu" "B.Cu") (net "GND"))
 (via (at 72 97.5) (size 1) (drill 0.5) (layers "F.Cu" "B.Cu") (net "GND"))
 (via (at 64 92.5) (size 1) (drill 0.5) (layers "F.Cu" "B.Cu") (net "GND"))
 (via (at 54.75 88.75) (size 0.6) (drill 0.3) (layers "F.Cu" "B.Cu") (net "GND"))
 (segment (start 92.8 38.3) (end 92.785 38.285) (width 1) (layer "B.Cu") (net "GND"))
 (segment (start 96.455 89.085) (end 82.085 89.085) (width 1) (layer "B.Cu") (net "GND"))
 (segment (start 59 84.5) (end 54.75 88.75) (width 1) (layer "B.Cu") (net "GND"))
 (segment (start 69 97.5) (end 72 97.5) (width 1) (layer "B.Cu") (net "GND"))
 (segment (start 64 92.5) (end 69 97.5) (width 1) (layer "B.Cu") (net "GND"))
 (segment (start 96 38.3) (end 92.8 38.3) (width 1) (layer "B.Cu") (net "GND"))
 (segment (start 92.785 38.285) (end 89.215 38.285) (width 1) (layer "B.Cu") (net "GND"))
 (segment (start 82 89) (end 82 45.5) (width 1) (layer "B.Cu") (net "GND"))
 (segment (start 82.085 89.085) (end 82 89) (width 1) (layer "B.Cu") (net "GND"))
 (segment (start 82 45.5) (end 89.215 38.285) (width 1) (layer "B.Cu") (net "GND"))
 (segment (start 95.955 41.545) (end 96 41.5) (width 1) (layer "B.Cu") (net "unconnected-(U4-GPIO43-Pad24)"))
 (segment (start 24 105.5) (end 31.5 98) (width 1) (layer "F.Cu") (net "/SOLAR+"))
 (segment (start 37.485 98) (end 37.685 98.2) (width 1) (layer "F.Cu") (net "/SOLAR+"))
 (segment (start 31.5 98) (end 37.485 98) (width 1) (layer "F.Cu") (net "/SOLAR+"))
 (segment (start 21.5 105.5) (end 24 105.5) (width 1) (layer "F.Cu") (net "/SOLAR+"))
 (segment (start 32 101) (end 38.839213 101) (width 1) (layer "F.Cu") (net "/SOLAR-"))
 (segment (start 38.839213 101) (end 40.5 99.339213) (width 1) (layer "F.Cu") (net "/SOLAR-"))
 (segment (start 24.96 108.04) (end 32 101) (width 1) (layer "F.Cu") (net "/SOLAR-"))
 (segment (start 21.5 108.04) (end 24.96 108.04) (width 1) (layer "F.Cu") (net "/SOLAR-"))
 (segment (start 40.5 99.339213) (end 40.5 98) (width 1) (layer "F.Cu") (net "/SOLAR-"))
 (segment (start 40.425 98) (end 40.225 98.2) (width 1) (layer "F.Cu") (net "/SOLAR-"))
 (segment (start 40.5 98) (end 40.425 98) (width 1) (layer "F.Cu") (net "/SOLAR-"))
 (segment (start 74 113) (end 74 115.5) (width 1) (layer "F.Cu") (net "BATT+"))
 (segment (start 69.275 111.045) (end 71.955 111.045) (width 1) (layer "F.Cu") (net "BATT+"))
 (segment (start 74 115.5) (end 71.5 118) (width 1) (layer "F.Cu") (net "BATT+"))
 (segment (start 45.505 98) (end 45.305 98.2) (width 1) (layer "F.Cu") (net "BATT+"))
 (segment (start 71.955 111.045) (end 72 111) (width 1) (layer "F.Cu") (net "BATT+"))
 (segment (start 71.5 118) (end 41 118) (width 1) (layer "F.Cu") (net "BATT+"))
 (segment (start 45.5 98.08) (end 45.58 98) (width 1) (layer "F.Cu") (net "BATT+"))
 (segment (start 22 118.04) (end 40.96 118.04) (width 1) (layer "F.Cu") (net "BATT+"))
 (segment (start 40.96 118.04) (end 45.5 113.5) (width 1) (layer "F.Cu") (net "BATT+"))
 (segment (start 41 118) (end 40.96 118.04) (width 1) (layer "F.Cu") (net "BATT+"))
 (segment (start 45.5 113.5) (end 45.5 98.08) (width 1) (layer "F.Cu") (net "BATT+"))
 (segment (start 45.58 98) (end 45.505 98) (width 1) (layer "F.Cu") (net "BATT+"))
 (segment (start 72 111) (end 74 113) (width 1) (layer "F.Cu") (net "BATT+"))
 (segment (start 43 98.435) (end 42.765 98.2) (width 1) (layer "F.Cu") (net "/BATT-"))
 (segment (start 22 115.5) (end 25 112.5) (width 1) (layer "F.Cu") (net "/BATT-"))
 (segment (start 39 112.5) (end 43 108.5) (width 1) (layer "F.Cu") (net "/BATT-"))
 (segment (start 25 112.5) (end 39 112.5) (width 1) (layer "F.Cu") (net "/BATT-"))
 (segment (start 43 108.5) (end 43 98.435) (width 1) (layer "F.Cu") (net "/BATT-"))
 (via (at 42.74 107.24) (size 0.6) (drill 0.3) (layers "F.Cu" "B.Cu") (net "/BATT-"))
 (segment (start 42.74 98.2) (end 43 98.46) (width 1) (layer "B.Cu") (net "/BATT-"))
 (segment (start 43 98.46) (end 43 106.98) (width 1) (layer "B.Cu") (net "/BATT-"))
 (segment (start 43 106.98) (end 43 107.5) (width 1) (layer "B.Cu") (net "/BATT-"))
 (segment (start 63 111) (end 65.495 108.505) (width 1) (layer "B.Cu") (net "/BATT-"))
 (segment (start 65.495 108.505) (end 69.275 108.505) (width 1) (layer "B.Cu") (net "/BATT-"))
 (segment (start 46.5 111) (end 63 111) (width 1) (layer "B.Cu") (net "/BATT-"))
 (segment (start 43 107.5) (end 46.5 111) (width 1) (layer "B.Cu") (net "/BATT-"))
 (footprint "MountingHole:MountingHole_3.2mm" (layer "F.Cu") (at 19.5 35.5)
  (pad "1" np_thru_hole circle (at 0 0) (size 3.2 3.2) (drill 3.2) (layers "*.Cu" "*.Mask")))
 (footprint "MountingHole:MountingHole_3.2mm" (layer "F.Cu") (at 107.5 35.5)
  (pad "1" np_thru_hole circle (at 0 0) (size 3.2 3.2) (drill 3.2) (layers "*.Cu" "*.Mask")))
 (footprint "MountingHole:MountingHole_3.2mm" (layer "F.Cu") (at 19.5 123.5)
  (pad "1" np_thru_hole circle (at 0 0) (size 3.2 3.2) (drill 3.2) (layers "*.Cu" "*.Mask")))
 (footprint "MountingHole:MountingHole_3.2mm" (layer "F.Cu") (at 107.5 123.5)
  (pad "1" np_thru_hole circle (at 0 0) (size 3.2 3.2) (drill 3.2) (layers "*.Cu" "*.Mask"))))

